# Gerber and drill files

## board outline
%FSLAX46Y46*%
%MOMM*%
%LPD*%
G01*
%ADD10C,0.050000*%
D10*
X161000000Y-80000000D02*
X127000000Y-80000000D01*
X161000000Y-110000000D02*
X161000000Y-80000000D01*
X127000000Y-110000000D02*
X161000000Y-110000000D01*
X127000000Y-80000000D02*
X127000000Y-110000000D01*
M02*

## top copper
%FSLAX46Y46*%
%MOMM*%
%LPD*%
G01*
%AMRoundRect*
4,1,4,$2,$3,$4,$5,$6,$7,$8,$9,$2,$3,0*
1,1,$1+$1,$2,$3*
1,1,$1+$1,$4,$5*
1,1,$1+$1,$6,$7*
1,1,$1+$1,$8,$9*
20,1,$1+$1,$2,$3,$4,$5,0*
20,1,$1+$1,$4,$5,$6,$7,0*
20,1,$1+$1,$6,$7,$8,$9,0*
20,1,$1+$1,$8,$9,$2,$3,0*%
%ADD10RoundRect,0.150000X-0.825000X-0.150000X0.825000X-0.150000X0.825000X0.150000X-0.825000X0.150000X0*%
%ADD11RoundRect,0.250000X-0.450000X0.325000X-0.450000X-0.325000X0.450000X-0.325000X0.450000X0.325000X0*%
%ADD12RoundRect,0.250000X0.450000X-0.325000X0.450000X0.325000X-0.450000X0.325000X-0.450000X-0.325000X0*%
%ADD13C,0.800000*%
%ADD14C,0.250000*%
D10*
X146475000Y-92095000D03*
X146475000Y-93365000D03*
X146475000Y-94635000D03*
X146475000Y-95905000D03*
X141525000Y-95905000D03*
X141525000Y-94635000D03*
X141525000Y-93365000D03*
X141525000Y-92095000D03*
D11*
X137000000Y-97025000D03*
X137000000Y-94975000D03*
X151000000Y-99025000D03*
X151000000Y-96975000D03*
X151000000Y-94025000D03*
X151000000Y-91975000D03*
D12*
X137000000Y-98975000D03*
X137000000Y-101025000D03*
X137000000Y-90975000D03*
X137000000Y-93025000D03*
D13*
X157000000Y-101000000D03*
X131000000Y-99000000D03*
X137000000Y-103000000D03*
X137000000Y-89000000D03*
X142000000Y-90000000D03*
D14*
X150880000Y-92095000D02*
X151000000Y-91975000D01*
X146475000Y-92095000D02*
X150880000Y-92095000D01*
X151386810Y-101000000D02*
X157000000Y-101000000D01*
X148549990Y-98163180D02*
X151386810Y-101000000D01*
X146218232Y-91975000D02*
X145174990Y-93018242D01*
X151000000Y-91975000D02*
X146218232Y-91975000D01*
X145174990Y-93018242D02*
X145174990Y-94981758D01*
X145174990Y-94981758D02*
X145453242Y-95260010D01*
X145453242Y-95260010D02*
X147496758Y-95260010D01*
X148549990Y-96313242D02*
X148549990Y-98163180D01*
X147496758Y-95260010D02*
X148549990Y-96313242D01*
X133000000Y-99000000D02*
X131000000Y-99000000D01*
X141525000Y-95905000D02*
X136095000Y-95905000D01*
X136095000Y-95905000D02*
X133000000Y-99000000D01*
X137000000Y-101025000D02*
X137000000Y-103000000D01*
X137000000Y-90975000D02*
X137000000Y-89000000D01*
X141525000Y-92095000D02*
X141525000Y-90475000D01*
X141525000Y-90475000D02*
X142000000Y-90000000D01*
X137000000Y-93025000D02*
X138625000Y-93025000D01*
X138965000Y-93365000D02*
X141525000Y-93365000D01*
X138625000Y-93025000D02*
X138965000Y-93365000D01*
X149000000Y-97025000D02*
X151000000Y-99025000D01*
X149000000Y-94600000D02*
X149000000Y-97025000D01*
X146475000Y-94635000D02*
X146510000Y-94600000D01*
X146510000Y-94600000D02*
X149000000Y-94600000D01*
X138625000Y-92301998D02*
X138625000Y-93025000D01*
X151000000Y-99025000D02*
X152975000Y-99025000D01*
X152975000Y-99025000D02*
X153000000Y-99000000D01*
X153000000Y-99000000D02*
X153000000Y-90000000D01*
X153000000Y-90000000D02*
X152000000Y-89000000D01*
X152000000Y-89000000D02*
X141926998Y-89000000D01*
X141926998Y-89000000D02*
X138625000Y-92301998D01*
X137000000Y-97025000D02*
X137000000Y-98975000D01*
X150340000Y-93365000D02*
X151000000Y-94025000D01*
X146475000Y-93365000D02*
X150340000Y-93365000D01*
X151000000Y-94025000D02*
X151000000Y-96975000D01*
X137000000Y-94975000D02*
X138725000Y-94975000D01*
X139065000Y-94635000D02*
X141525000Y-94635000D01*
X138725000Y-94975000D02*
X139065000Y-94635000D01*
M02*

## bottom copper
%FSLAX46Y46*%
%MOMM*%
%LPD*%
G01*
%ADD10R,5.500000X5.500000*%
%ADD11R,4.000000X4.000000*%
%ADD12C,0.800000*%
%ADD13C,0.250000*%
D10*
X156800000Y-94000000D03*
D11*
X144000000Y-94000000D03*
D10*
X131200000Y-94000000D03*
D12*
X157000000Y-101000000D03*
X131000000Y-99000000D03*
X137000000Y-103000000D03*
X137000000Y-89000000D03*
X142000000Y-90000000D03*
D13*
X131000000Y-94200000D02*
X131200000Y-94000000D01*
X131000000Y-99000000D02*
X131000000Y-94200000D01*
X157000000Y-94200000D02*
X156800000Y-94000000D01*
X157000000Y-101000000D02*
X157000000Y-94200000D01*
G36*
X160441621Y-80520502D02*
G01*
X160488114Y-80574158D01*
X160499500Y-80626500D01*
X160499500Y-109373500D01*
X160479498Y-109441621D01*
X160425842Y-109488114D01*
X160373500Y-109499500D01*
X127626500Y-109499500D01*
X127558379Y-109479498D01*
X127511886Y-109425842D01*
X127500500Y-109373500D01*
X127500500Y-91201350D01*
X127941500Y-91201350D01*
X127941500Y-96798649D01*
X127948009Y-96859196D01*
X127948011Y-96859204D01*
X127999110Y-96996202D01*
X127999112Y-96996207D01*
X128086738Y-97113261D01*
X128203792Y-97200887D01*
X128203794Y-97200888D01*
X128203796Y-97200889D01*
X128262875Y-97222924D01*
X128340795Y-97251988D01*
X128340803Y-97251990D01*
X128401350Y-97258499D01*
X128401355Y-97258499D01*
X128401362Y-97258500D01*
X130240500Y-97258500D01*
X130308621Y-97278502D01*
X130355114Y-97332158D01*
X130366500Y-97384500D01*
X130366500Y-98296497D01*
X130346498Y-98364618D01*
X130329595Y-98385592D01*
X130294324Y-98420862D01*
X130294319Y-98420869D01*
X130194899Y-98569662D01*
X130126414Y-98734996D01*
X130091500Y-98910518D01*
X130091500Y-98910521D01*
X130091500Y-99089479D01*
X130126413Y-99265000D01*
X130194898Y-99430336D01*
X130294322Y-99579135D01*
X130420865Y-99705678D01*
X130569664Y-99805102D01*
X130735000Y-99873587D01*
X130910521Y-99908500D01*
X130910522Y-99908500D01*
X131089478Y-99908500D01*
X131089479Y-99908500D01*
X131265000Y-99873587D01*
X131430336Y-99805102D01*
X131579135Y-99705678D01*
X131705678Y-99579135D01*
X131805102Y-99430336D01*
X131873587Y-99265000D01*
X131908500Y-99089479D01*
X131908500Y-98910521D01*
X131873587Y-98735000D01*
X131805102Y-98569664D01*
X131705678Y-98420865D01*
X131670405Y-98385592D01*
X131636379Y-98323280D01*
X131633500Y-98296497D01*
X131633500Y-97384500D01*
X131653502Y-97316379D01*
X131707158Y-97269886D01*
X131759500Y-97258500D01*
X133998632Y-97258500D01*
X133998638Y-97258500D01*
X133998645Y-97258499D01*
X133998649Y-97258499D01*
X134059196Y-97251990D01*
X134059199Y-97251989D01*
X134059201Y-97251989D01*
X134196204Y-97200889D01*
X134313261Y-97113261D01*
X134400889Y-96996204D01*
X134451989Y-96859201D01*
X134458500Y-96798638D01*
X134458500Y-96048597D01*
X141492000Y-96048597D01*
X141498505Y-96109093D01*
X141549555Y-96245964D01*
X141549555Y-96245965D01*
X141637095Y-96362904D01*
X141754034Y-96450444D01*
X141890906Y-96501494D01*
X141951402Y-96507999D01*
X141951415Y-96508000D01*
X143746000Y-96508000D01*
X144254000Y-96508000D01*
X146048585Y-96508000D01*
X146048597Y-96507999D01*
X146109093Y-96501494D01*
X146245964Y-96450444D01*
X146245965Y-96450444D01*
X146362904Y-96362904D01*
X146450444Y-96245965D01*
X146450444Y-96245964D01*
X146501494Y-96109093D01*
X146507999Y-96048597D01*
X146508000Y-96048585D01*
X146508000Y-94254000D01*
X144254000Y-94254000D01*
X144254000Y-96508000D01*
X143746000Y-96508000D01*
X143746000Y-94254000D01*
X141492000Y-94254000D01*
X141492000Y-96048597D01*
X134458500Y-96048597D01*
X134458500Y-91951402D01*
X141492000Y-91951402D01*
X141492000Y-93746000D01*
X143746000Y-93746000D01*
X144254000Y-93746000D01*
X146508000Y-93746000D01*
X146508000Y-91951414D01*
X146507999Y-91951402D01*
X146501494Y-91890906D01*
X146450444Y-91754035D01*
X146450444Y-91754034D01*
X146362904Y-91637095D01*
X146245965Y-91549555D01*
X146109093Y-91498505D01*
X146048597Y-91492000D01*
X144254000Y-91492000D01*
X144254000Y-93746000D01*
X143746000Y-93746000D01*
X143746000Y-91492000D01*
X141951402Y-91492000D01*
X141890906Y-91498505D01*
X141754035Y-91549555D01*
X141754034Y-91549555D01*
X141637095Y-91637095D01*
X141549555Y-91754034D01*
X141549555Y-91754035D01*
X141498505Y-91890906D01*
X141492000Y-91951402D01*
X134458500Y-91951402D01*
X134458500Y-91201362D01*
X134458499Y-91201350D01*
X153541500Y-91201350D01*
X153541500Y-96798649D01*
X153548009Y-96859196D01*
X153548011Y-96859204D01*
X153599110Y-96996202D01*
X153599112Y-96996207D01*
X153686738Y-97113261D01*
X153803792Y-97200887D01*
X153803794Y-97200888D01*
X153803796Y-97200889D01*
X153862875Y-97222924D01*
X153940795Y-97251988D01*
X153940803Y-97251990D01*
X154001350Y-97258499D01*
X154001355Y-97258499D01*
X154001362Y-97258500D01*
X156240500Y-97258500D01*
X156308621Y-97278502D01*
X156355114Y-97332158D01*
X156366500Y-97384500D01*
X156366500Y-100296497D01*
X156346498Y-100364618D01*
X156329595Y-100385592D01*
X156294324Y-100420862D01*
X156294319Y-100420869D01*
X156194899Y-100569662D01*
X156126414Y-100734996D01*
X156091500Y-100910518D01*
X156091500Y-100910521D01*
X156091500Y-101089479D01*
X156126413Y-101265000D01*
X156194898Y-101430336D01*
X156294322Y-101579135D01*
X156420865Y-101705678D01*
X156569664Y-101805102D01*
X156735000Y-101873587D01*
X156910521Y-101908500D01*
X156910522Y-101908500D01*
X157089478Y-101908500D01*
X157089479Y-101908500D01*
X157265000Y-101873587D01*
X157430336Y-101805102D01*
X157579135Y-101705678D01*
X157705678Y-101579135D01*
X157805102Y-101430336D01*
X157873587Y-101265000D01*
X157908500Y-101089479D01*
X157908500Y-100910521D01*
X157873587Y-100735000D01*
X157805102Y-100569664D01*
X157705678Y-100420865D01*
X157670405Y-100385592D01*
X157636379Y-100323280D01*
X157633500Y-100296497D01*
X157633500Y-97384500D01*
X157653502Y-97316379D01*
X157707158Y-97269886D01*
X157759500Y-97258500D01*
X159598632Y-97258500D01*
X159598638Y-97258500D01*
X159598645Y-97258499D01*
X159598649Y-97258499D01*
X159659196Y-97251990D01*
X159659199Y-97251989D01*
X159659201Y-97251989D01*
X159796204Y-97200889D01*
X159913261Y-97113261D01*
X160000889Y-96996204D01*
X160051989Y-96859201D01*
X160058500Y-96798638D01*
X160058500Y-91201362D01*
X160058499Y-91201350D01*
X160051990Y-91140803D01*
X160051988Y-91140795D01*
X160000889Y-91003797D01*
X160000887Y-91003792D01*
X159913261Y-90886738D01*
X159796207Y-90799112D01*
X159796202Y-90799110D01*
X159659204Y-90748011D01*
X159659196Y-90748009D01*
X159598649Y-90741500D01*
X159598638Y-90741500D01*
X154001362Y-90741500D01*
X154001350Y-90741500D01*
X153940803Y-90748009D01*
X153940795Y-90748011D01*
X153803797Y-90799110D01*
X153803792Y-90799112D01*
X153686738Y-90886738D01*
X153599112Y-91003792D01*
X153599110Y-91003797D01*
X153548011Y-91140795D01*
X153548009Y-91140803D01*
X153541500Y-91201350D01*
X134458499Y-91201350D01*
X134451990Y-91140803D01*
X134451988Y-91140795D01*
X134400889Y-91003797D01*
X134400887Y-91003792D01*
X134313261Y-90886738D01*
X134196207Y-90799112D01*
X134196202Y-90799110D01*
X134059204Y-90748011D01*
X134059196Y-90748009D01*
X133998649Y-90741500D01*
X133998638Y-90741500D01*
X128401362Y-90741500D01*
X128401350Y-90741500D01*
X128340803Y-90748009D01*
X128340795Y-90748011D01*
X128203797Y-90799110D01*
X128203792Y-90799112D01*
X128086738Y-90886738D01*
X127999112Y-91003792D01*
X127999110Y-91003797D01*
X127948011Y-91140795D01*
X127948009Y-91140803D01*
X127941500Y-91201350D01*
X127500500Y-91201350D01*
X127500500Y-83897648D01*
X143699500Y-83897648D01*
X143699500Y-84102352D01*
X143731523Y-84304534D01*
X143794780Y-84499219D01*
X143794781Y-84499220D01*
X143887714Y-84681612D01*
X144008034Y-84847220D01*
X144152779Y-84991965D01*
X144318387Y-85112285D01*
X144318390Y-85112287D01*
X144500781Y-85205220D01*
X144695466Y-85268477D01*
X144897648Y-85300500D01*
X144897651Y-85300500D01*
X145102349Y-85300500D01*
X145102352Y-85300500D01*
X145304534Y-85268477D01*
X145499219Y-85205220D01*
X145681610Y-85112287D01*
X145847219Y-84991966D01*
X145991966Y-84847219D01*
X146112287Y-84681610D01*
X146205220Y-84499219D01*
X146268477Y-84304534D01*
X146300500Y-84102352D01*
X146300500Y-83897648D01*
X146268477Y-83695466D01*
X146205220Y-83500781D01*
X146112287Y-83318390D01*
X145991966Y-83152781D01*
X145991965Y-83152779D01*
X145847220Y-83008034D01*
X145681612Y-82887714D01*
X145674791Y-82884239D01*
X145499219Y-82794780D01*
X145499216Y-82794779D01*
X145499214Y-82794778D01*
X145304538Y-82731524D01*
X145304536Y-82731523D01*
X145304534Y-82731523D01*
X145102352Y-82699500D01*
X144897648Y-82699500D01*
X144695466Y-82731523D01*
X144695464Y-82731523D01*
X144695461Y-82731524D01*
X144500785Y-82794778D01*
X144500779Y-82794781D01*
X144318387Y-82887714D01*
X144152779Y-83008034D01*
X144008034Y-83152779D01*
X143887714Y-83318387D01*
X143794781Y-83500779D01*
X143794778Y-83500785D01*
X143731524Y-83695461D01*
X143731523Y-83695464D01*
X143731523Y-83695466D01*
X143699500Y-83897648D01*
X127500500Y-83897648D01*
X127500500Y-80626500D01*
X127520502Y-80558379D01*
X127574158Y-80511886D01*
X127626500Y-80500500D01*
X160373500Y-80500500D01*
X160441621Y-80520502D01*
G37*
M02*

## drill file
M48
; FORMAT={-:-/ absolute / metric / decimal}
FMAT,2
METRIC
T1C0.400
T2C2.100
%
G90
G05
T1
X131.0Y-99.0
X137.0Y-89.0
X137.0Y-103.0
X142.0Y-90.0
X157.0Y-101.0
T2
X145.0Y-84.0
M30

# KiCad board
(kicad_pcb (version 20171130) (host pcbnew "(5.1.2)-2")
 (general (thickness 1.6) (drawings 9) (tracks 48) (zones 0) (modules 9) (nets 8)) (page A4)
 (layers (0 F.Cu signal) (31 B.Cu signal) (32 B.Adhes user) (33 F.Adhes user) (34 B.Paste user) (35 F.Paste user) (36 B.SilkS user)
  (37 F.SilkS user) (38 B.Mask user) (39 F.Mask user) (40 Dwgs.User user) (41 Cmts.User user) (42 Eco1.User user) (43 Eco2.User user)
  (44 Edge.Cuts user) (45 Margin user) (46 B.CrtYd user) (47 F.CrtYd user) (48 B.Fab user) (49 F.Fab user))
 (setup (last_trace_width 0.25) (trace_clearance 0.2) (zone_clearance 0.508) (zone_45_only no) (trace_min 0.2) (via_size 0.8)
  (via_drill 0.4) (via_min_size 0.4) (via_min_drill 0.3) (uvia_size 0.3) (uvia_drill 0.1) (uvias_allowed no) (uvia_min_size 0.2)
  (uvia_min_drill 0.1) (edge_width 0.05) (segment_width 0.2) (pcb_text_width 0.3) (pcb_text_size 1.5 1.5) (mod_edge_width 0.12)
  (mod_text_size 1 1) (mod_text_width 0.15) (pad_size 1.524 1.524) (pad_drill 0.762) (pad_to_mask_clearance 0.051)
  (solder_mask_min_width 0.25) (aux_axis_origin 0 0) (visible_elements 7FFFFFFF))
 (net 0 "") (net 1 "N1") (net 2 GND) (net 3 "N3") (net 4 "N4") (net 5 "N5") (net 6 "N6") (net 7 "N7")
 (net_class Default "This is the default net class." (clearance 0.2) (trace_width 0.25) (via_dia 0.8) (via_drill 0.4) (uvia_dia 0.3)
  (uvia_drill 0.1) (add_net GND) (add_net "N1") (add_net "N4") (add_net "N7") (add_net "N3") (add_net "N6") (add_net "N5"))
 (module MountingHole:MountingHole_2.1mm (layer F.Cu) (at 145 84)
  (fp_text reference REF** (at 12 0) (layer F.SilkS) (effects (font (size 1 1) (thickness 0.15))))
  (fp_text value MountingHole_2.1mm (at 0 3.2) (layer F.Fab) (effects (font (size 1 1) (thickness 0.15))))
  (pad "" np_thru_hole circle (at 0 0) (size 2.1 2.1) (drill 2.1) (layers *.Cu *.Mask)))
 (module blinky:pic (layer F.Cu) (at 134 85)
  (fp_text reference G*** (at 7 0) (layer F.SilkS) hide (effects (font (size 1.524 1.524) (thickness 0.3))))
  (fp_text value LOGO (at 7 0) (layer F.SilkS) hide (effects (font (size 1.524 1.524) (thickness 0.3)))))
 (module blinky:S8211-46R (layer B.Cu) (at 144 94)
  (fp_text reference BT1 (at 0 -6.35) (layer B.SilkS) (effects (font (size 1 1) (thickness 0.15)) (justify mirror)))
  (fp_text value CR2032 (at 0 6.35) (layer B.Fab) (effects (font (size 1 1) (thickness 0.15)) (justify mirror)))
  (pad 1 smd rect (at 12.8 0) (size 5.5 5.5) (layers B.Cu B.Paste B.Mask) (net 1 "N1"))
  (pad 2 smd rect (at 0 0) (size 4 4) (layers B.Cu B.Paste B.Mask) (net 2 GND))
  (pad 1 smd rect (at -12.8 0) (size 5.5 5.5) (layers B.Cu B.Paste B.Mask) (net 1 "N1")))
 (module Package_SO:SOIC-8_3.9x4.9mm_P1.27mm (layer F.Cu) (at 144 94)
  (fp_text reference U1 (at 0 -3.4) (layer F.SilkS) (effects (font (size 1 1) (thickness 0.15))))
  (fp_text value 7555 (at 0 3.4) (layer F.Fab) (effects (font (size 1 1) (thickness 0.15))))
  (pad 8 smd roundrect (at 2.475 -1.905) (size 1.95 0.6) (layers F.Cu F.Paste F.Mask) (roundrect_rratio 0.25) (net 1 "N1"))
  (pad 7 smd roundrect (at 2.475 -0.635) (size 1.95 0.6) (layers F.Cu F.Paste F.Mask) (roundrect_rratio 0.25) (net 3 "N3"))
  (pad 6 smd roundrect (at 2.475 0.635) (size 1.95 0.6) (layers F.Cu F.Paste F.Mask) (roundrect_rratio 0.25) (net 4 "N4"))
  (pad 5 smd roundrect (at 2.475 1.905) (size 1.95 0.6) (layers F.Cu F.Paste F.Mask) (roundrect_rratio 0.25) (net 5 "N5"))
  (pad 4 smd roundrect (at -2.475 1.905) (size 1.95 0.6) (layers F.Cu F.Paste F.Mask) (roundrect_rratio 0.25) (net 1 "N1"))
  (pad 3 smd roundrect (at -2.475 0.635) (size 1.95 0.6) (layers F.Cu F.Paste F.Mask) (roundrect_rratio 0.25) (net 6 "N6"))
  (pad 2 smd roundrect (at -2.475 -0.635) (size 1.95 0.6) (layers F.Cu F.Paste F.Mask) (roundrect_rratio 0.25) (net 4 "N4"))
  (pad 1 smd roundrect (at -2.475 -1.905) (size 1.95 0.6) (layers F.Cu F.Paste F.Mask) (roundrect_rratio 0.25) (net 2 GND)))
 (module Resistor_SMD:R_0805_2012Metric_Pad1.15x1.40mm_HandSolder (layer F.Cu) (at 137 96 270)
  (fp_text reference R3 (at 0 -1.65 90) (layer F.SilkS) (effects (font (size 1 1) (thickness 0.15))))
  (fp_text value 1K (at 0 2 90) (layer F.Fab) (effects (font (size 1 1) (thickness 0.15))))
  (pad 2 smd roundrect (at 1.025 0 270) (size 1.15 1.4) (layers F.Cu F.Paste F.Mask) (roundrect_rratio 0.217391) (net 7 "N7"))
  (pad 1 smd roundrect (at -1.025 0 270) (size 1.15 1.4) (layers F.Cu F.Paste F.Mask) (roundrect_rratio 0.217391) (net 6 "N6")))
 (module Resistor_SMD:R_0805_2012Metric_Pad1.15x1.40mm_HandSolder (layer F.Cu) (at 151 98 270)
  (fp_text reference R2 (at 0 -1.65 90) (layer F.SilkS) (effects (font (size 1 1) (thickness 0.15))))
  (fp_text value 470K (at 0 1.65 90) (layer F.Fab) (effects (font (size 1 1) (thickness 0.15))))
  (pad 2 smd roundrect (at 1.025 0 270) (size 1.15 1.4) (layers F.Cu F.Paste F.Mask) (roundrect_rratio 0.217391) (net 4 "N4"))
  (pad 1 smd roundrect (at -1.025 0 270) (size 1.15 1.4) (layers F.Cu F.Paste F.Mask) (roundrect_rratio 0.217391) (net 3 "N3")))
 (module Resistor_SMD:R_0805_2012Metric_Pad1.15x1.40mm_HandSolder (layer F.Cu) (at 151 93 270)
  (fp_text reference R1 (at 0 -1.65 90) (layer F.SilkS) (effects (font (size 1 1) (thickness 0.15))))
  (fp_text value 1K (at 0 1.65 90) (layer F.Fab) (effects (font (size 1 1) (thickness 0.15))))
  (pad 2 smd roundrect (at 1.025 0 270) (size 1.15 1.4) (layers F.Cu F.Paste F.Mask) (roundrect_rratio 0.217391) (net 3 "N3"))
  (pad 1 smd roundrect (at -1.025 0 270) (size 1.15 1.4) (layers F.Cu F.Paste F.Mask) (roundrect_rratio 0.217391) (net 1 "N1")))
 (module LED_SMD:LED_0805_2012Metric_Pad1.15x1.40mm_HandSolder (layer F.Cu) (at 137 100 90)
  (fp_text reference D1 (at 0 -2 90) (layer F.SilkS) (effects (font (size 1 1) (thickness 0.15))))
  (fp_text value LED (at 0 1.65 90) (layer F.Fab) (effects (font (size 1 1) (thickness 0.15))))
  (pad 2 smd roundrect (at 1.025 0 90) (size 1.15 1.4) (layers F.Cu F.Paste F.Mask) (roundrect_rratio 0.217391) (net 7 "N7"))
  (pad 1 smd roundrect (at -1.025 0 90) (size 1.15 1.4) (layers F.Cu F.Paste F.Mask) (roundrect_rratio 0.217391) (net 2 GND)))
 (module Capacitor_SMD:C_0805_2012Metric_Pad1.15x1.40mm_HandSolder (layer F.Cu) (at 137 92 90)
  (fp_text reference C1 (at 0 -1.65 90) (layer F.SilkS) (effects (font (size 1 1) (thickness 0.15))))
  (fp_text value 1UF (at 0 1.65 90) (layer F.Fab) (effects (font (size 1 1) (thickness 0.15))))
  (pad 2 smd roundrect (at 1.025 0 90) (size 1.15 1.4) (layers F.Cu F.Paste F.Mask) (roundrect_rratio 0.217391) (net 2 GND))
  (pad 1 smd roundrect (at -1.025 0 90) (size 1.15 1.4) (layers F.Cu F.Paste F.Mask) (roundrect_rratio 0.217391) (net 4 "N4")))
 (gr_line (start 161 80) (end 127 80) (layer Edge.Cuts) (width 0.05))
 (gr_line (start 161 110) (end 161 80) (layer Edge.Cuts) (width 0.05))
 (gr_line (start 127 110) (end 161 110) (layer Edge.Cuts) (width 0.05))
 (gr_line (start 127 80) (end 127 110) (layer Edge.Cuts) (width 0.05))
 (segment (start 150.88 92.095) (end 151 91.975) (width 0.25) (layer F.Cu) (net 1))
 (segment (start 146.475 92.095) (end 150.88 92.095) (width 0.25) (layer F.Cu) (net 1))
 (via (at 157 101) (size 0.8) (drill 0.4) (layers F.Cu B.Cu) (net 1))
 (segment (start 151.38681 101) (end 157 101) (width 0.25) (layer F.Cu) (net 1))
 (segment (start 148.54999 98.16318) (end 151.38681 101) (width 0.25) (layer F.Cu) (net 1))
 (segment (start 146.218232 91.975) (end 145.17499 93.018242) (width 0.25) (layer F.Cu) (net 1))
 (segment (start 151 91.975) (end 146.218232 91.975) (width 0.25) (layer F.Cu) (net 1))
 (segment (start 145.17499 93.018242) (end 145.17499 94.981758) (width 0.25) (layer F.Cu) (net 1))
 (segment (start 145.17499 94.981758) (end 145.453242 95.26001) (width 0.25) (layer F.Cu) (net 1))
 (segment (start 145.453242 95.26001) (end 147.496758 95.26001) (width 0.25) (layer F.Cu) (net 1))
 (segment (start 148.54999 96.313242) (end 148.54999 98.16318) (width 0.25) (layer F.Cu) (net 1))
 (segment (start 147.496758 95.26001) (end 148.54999 96.313242) (width 0.25) (layer F.Cu) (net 1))
 (via (at 131 99) (size 0.8) (drill 0.4) (layers F.Cu B.Cu) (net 1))
 (segment (start 131 94.2) (end 131.2 94) (width 0.25) (layer B.Cu) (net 1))
 (segment (start 131 99) (end 131 94.2) (width 0.25) (layer B.Cu) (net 1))
 (segment (start 157 94.2) (end 156.8 94) (width 0.25) (layer B.Cu) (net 1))
 (segment (start 157 101) (end 157 94.2) (width 0.25) (layer B.Cu) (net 1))
 (segment (start 133 99) (end 131 99) (width 0.25) (layer F.Cu) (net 1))
 (segment (start 141.525 95.905) (end 136.095 95.905) (width 0.25) (layer F.Cu) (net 1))
 (segment (start 136.095 95.905) (end 133 99) (width 0.25) (layer F.Cu) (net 1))
 (via (at 137 103) (size 0.8) (drill 0.4) (layers F.Cu B.Cu) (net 2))
 (segment (start 137 101.025) (end 137 103) (width 0.25) (layer F.Cu) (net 2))
 (via (at 137 89) (size 0.8) (drill 0.4) (layers F.Cu B.Cu) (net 2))
 (segment (start 137 90.975) (end 137 89) (width 0.25) (layer F.Cu) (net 2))
 (via (at 142 90) (size 0.8) (drill 0.4) (layers F.Cu B.Cu) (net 2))
 (segment (start 141.525 92.095) (end 141.525 90.475) (width 0.25) (layer F.Cu) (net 2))
 (segment (start 141.525 90.475) (end 142 90) (width 0.25) (layer F.Cu) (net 2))
 (segment (start 137 93.025) (end 138.625 93.025) (width 0.25) (layer F.Cu) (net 4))
 (segment (start 138.965 93.365) (end 141.525 93.365) (width 0.25) (layer F.Cu) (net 4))
 (segment (start 138.625 93.025) (end 138.965 93.365) (width 0.25) (layer F.Cu) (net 4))
 (segment (start 149 97.025) (end 151 99.025) (width 0.25) (layer F.Cu) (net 4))
 (segment (start 149 94.6) (end 149 97.025) (width 0.25) (layer F.Cu) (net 4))
 (segment (start 146.475 94.635) (end 146.51 94.6) (width 0.25) (layer F.Cu) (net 4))
 (segment (start 146.51 94.6) (end 149 94.6) (width 0.25) (layer F.Cu) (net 4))
 (segment (start 138.625 92.301998) (end 138.625 93.025) (width 0.25) (layer F.Cu) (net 4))
 (segment (start 151 99.025) (end 152.975 99.025) (width 0.25) (layer F.Cu) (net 4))
 (segment (start 152.975 99.025) (end 153 99) (width 0.25) (layer F.Cu) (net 4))
 (segment (start 153 99) (end 153 90) (width 0.25) (layer F.Cu) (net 4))
 (segment (start 153 90) (end 152 89) (width 0.25) (layer F.Cu) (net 4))
 (segment (start 152 89) (end 141.926998 89) (width 0.25) (layer F.Cu) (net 4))
 (segment (start 141.926998 89) (end 138.625 92.301998) (width 0.25) (layer F.Cu) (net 4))
 (segment (start 137 97.025) (end 137 98.975) (width 0.25) (layer F.Cu) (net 7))
 (segment (start 150.34 93.365) (end 151 94.025) (width 0.25) (layer F.Cu) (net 3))
 (segment (start 146.475 93.365) (end 150.34 93.365) (width 0.25) (layer F.Cu) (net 3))
 (segment (start 151 94.025) (end 151 96.975) (width 0.25) (layer F.Cu) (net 3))
 (segment (start 137 94.975) (end 138.725 94.975) (width 0.25) (layer F.Cu) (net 6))
 (segment (start 139.065 94.635) (end 141.525 94.635) (width 0.25) (layer F.Cu) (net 6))
 (segment (start 138.725 94.975) (end 139.065 94.635) (width 0.25) (layer F.Cu) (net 6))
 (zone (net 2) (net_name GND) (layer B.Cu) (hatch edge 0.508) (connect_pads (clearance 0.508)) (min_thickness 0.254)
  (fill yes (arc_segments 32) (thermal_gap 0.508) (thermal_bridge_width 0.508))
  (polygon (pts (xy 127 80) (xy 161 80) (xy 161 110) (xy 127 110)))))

